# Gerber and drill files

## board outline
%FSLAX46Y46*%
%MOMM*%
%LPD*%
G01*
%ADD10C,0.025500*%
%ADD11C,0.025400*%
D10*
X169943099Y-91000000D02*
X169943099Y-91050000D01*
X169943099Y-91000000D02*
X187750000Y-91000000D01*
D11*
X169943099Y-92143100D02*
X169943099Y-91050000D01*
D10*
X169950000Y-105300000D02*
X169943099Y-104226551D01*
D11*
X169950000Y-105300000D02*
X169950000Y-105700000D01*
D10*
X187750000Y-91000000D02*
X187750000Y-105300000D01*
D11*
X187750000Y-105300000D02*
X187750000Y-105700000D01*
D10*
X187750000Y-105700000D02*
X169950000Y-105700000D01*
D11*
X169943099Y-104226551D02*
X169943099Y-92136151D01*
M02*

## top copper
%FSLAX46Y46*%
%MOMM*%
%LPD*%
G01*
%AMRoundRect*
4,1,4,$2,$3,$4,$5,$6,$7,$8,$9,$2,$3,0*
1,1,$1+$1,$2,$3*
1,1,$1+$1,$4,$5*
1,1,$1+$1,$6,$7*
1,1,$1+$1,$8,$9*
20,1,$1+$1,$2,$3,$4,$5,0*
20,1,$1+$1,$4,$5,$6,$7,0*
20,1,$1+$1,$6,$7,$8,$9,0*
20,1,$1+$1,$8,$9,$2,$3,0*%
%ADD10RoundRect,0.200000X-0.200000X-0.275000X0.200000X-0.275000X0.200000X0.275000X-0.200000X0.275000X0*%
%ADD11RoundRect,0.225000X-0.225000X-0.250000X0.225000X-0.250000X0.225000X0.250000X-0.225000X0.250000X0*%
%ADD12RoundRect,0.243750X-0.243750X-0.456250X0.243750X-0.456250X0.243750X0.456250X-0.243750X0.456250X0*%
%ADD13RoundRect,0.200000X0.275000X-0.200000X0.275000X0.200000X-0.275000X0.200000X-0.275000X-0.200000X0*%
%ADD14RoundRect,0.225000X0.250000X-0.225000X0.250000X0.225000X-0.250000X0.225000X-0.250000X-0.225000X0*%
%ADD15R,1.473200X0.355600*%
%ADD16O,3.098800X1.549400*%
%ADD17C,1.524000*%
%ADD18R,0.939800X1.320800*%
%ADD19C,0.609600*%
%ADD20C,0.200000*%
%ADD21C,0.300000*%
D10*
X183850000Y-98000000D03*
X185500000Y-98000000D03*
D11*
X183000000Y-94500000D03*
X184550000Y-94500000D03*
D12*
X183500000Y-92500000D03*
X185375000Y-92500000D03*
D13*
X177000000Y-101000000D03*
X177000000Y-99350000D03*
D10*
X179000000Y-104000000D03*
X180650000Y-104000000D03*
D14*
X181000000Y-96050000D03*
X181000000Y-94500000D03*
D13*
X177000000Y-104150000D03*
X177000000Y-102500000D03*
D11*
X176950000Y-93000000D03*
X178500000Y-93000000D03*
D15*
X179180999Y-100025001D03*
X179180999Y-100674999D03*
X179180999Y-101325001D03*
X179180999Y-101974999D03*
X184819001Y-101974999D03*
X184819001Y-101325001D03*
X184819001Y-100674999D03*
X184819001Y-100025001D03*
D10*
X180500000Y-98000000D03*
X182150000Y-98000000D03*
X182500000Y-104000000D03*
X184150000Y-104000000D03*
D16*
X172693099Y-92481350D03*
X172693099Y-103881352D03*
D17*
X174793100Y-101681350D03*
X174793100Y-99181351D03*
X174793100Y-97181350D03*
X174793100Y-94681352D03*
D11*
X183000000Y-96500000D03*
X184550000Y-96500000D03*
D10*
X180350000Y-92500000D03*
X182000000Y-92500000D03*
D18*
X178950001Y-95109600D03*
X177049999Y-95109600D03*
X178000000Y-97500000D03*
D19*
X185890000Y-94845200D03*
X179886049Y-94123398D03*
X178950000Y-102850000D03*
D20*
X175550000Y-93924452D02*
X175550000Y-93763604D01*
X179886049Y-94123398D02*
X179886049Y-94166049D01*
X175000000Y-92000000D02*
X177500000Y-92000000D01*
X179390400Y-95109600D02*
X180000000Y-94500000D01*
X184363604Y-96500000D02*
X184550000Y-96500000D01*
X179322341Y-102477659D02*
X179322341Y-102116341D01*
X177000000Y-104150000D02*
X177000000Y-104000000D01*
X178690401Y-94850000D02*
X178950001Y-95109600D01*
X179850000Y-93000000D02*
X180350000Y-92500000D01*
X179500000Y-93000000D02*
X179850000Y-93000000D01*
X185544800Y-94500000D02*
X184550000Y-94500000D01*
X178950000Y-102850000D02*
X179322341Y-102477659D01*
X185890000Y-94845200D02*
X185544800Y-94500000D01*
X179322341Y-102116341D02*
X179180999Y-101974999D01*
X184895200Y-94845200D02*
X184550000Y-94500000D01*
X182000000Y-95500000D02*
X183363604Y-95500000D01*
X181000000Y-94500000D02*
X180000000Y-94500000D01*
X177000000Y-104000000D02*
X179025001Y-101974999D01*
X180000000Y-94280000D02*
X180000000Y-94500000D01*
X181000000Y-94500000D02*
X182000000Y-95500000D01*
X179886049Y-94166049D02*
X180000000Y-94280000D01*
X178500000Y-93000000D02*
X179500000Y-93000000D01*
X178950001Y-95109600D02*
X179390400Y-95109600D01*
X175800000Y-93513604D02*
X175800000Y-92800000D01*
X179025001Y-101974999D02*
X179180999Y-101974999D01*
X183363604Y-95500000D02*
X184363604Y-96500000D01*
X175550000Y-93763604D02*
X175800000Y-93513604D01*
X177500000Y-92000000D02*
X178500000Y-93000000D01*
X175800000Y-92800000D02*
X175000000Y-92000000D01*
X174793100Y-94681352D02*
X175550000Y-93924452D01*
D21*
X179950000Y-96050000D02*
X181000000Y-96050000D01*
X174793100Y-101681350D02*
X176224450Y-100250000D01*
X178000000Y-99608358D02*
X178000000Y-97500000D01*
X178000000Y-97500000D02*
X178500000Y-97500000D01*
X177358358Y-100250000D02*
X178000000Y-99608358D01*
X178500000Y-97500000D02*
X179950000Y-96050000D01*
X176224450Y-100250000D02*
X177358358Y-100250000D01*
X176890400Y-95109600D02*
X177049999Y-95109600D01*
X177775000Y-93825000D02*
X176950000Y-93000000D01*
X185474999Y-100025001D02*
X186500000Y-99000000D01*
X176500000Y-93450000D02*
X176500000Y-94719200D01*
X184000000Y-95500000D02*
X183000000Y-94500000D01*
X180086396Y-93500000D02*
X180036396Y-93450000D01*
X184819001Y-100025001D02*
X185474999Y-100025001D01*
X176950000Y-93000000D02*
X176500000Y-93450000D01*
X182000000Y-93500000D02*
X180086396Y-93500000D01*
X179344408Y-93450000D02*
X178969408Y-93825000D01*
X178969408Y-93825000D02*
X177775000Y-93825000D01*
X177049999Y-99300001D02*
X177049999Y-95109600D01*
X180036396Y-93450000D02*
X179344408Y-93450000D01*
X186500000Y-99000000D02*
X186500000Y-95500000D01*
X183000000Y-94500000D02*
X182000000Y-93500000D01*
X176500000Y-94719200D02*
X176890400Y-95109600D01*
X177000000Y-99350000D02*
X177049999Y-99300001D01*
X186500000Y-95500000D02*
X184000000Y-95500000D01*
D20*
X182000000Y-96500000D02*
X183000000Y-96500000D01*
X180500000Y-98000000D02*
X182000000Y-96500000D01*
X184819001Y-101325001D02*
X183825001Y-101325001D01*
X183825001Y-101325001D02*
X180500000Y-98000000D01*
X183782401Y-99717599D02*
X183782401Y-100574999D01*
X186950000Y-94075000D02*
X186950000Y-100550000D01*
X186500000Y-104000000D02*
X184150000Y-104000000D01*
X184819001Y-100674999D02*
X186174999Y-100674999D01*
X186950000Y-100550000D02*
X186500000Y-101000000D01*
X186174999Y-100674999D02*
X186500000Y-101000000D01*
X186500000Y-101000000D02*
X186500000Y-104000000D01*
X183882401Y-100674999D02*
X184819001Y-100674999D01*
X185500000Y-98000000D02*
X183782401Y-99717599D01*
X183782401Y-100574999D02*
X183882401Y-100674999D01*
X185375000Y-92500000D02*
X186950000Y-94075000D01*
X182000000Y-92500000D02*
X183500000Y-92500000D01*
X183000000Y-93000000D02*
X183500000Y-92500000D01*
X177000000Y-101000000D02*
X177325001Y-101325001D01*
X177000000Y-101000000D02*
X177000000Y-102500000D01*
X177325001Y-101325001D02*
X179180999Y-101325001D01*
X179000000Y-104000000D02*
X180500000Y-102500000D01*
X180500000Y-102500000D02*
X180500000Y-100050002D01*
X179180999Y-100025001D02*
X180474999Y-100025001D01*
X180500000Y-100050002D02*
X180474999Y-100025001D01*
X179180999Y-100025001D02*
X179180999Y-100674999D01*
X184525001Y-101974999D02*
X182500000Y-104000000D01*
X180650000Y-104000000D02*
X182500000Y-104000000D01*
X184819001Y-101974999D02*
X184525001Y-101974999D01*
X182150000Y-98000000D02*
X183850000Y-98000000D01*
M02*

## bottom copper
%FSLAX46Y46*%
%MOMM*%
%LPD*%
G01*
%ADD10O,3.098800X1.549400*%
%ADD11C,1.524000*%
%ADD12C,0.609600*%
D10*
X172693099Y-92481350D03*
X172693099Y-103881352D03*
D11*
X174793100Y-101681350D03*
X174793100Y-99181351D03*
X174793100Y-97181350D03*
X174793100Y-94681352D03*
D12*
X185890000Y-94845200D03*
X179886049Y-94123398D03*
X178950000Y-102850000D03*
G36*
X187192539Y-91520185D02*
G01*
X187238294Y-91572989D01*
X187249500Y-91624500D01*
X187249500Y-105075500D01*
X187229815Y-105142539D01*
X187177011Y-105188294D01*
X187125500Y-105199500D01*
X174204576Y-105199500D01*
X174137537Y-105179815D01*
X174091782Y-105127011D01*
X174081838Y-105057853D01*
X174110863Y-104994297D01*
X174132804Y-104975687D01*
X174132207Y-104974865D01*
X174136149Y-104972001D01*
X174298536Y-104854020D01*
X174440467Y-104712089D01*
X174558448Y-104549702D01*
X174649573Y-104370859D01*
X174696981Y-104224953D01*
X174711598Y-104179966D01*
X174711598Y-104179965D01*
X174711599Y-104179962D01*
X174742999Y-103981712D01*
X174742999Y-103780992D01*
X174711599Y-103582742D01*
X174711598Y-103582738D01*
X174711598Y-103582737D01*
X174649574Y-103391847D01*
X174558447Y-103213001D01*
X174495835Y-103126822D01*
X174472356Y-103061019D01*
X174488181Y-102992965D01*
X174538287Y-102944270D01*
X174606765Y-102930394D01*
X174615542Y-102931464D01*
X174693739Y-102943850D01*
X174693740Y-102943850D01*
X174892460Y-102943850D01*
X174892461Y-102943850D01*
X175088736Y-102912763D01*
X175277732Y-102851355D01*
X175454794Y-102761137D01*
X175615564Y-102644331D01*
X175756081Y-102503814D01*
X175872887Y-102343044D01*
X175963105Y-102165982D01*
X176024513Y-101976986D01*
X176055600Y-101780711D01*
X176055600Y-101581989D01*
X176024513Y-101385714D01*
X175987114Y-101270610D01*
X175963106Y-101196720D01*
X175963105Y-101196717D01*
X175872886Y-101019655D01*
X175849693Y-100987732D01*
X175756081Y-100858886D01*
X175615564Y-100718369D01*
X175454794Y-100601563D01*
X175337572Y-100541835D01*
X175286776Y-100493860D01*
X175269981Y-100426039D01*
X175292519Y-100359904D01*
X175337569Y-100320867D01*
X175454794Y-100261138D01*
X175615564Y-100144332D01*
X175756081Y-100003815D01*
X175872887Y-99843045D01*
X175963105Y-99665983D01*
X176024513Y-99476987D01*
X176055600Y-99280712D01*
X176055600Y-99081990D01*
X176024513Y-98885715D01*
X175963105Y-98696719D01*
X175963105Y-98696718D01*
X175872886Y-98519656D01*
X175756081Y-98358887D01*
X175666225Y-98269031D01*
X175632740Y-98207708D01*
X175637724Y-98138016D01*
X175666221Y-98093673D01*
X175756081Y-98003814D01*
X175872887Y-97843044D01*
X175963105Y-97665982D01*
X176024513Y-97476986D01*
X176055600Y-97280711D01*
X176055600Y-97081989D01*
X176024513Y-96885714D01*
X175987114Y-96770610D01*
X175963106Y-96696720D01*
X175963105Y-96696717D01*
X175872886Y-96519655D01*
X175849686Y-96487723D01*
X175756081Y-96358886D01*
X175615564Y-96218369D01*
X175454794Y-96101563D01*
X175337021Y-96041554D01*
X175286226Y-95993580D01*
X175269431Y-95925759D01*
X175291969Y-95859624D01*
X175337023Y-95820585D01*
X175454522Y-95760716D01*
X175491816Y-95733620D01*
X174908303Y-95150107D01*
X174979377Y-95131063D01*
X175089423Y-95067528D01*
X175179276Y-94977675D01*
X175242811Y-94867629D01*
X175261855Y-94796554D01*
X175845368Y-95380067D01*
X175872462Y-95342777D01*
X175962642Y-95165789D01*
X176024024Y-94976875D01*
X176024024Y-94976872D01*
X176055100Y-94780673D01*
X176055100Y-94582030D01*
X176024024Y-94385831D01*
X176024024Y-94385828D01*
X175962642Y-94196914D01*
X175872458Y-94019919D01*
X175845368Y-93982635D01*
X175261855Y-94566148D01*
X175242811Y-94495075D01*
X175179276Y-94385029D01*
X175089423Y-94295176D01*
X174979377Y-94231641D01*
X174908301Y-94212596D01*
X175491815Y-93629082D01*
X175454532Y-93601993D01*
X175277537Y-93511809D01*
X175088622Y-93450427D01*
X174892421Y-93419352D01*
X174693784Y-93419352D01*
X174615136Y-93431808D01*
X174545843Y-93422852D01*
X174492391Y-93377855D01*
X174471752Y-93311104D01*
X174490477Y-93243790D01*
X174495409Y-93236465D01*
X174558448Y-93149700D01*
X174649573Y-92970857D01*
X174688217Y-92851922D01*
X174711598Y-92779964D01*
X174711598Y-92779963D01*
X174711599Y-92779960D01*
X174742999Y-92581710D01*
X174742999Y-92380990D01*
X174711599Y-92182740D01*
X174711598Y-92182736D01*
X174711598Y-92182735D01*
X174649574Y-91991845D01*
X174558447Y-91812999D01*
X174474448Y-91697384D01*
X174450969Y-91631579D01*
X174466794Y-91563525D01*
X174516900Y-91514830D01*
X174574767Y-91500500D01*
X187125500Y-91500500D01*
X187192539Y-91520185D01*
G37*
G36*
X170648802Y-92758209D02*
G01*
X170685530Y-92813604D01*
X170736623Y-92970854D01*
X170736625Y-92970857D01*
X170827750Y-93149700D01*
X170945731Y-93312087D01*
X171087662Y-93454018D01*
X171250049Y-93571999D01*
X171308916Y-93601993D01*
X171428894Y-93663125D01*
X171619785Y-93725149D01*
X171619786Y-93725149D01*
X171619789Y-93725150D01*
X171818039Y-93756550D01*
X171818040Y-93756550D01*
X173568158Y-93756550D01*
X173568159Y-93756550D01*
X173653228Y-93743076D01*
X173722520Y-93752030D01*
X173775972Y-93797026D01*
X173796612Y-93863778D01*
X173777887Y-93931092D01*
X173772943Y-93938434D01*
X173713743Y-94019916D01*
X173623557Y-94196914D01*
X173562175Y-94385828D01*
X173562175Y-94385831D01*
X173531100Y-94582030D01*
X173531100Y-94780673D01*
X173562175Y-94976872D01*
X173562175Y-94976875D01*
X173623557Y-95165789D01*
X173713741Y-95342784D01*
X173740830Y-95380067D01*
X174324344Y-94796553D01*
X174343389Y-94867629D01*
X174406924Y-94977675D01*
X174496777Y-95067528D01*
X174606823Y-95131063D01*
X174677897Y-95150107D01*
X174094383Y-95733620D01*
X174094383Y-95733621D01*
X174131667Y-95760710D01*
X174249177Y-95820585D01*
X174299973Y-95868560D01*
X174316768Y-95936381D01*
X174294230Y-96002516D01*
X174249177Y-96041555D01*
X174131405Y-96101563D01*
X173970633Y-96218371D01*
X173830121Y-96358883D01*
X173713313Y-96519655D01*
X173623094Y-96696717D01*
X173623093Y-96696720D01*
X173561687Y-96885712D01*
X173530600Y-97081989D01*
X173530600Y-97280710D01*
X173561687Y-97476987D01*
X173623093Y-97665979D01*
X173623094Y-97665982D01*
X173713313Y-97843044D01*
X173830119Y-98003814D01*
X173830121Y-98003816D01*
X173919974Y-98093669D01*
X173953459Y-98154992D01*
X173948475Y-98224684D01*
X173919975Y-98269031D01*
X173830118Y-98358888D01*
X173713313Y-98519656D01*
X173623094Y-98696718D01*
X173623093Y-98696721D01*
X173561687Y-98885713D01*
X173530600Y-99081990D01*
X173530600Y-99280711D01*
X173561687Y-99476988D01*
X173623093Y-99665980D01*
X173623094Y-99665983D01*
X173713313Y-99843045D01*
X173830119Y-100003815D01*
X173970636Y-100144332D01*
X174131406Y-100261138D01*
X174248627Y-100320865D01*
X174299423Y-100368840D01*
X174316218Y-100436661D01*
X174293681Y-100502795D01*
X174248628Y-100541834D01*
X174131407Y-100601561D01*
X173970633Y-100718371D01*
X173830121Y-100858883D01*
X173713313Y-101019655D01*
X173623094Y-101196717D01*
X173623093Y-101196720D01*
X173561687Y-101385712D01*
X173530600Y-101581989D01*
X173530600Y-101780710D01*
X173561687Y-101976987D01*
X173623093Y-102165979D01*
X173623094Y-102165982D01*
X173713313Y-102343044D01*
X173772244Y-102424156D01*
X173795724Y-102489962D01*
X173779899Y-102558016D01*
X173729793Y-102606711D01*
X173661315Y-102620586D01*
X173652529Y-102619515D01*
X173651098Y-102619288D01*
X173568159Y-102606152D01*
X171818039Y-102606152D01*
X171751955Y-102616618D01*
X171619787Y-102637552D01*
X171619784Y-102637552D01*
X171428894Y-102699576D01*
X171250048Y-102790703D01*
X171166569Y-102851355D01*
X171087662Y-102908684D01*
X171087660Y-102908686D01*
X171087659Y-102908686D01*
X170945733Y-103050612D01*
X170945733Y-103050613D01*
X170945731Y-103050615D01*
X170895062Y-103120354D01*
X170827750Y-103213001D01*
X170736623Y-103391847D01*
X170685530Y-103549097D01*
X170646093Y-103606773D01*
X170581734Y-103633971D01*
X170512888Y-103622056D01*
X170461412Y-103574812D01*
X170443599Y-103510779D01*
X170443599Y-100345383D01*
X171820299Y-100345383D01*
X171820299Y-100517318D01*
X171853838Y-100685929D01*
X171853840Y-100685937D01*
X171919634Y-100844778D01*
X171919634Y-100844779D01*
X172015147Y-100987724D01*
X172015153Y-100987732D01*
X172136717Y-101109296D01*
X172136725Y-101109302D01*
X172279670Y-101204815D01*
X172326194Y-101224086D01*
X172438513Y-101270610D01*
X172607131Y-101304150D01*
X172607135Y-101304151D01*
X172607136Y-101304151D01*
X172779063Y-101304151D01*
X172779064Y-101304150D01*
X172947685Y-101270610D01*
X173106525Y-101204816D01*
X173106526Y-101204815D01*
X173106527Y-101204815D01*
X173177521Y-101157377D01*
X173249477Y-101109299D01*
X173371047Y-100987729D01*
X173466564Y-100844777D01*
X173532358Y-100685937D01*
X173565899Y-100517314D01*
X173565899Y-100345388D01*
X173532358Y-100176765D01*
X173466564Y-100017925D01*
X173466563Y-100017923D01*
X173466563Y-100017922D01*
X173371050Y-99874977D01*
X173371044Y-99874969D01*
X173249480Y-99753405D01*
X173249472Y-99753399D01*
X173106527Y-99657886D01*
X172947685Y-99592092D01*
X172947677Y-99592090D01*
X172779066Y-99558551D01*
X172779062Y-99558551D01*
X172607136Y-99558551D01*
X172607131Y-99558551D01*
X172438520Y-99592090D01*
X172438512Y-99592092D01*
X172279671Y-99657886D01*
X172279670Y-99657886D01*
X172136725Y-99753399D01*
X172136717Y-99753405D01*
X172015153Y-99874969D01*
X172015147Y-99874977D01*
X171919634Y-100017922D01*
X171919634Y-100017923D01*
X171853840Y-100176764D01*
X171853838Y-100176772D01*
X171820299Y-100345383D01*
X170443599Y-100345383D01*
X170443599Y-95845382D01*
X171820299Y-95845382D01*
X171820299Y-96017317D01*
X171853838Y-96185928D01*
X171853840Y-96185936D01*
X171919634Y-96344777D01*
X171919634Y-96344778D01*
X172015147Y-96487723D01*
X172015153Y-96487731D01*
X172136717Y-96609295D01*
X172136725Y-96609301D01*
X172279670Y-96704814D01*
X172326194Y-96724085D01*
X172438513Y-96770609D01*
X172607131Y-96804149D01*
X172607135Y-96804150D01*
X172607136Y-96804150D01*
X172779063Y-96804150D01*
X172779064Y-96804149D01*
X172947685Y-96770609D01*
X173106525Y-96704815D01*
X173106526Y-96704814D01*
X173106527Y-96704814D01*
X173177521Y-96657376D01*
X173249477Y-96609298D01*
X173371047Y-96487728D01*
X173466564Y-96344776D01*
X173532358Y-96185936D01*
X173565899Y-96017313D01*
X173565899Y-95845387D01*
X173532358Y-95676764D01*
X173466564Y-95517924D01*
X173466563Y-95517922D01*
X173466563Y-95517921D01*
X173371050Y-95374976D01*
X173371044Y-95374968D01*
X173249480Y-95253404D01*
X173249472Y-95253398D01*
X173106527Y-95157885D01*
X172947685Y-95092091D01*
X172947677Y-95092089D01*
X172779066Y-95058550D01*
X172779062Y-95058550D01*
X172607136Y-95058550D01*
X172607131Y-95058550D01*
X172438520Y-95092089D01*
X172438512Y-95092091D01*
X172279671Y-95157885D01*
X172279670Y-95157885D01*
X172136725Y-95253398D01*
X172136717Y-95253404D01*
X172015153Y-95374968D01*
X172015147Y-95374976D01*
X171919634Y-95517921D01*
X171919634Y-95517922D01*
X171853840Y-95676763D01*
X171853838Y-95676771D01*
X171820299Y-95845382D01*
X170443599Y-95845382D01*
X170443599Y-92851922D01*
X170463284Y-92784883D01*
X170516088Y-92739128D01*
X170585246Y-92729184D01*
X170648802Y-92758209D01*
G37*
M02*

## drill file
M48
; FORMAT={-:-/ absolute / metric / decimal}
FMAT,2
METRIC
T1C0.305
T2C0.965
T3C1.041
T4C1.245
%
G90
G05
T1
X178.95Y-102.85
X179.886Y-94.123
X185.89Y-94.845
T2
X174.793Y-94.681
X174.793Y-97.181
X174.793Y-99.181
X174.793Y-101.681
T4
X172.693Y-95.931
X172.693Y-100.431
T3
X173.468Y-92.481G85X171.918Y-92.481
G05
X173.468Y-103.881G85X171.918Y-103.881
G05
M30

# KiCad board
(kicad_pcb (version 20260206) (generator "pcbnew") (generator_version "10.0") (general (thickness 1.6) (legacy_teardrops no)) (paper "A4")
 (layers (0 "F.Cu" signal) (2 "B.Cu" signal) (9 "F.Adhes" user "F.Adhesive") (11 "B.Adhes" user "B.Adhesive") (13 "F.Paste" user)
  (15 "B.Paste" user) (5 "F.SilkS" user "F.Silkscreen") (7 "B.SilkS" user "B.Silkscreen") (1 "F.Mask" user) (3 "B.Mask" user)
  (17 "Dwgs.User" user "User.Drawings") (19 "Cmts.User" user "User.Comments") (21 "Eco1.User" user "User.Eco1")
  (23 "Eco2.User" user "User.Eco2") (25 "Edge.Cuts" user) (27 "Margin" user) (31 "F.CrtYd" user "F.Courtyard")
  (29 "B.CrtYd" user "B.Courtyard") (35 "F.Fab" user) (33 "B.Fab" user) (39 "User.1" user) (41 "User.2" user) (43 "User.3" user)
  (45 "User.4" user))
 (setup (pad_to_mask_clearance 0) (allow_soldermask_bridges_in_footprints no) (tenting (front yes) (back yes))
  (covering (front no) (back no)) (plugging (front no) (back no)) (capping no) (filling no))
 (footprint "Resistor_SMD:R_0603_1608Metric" (layer "F.Cu") (at 184.675 98)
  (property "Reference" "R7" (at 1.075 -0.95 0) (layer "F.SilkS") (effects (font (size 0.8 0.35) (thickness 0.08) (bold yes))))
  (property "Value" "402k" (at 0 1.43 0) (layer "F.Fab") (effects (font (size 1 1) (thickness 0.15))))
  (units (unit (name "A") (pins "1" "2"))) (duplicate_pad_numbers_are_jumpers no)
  (pad "1" smd roundrect (at -0.825 0) (size 0.8 0.95) (layers "F.Cu" "F.Mask" "F.Paste") (roundrect_rratio 0.25) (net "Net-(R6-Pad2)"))
  (pad "2" smd roundrect (at 0.825 0) (size 0.8 0.95) (layers "F.Cu" "F.Mask" "F.Paste") (roundrect_rratio 0.25) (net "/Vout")))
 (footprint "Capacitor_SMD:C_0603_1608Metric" (layer "F.Cu") (at 183.775 94.5)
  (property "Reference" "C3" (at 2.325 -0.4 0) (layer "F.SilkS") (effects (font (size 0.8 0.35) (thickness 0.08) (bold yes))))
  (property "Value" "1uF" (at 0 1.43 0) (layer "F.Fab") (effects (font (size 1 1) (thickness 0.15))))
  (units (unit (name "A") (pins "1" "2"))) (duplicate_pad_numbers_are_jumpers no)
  (pad "1" smd roundrect (at -0.775 0) (size 0.9 0.95) (layers "F.Cu" "F.Mask" "F.Paste") (roundrect_rratio 0.25) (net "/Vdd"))
  (pad "2" smd roundrect (at 0.775 0) (size 0.9 0.95) (layers "F.Cu" "F.Mask" "F.Paste") (roundrect_rratio 0.25) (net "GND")))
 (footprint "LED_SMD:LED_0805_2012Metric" (layer "F.Cu") (at 184.4375 92.5)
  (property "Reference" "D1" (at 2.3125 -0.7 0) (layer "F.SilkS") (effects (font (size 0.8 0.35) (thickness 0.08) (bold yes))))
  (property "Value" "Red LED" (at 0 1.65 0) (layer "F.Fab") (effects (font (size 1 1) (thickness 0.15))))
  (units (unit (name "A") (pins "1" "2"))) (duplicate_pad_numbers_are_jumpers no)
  (pad "1" smd roundrect (at -0.9375 0) (size 0.975 1.4) (layers "F.Cu" "F.Mask" "F.Paste") (roundrect_rratio 0.25) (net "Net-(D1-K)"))
  (pad "2" smd roundrect (at 0.9375 0) (size 0.975 1.4) (layers "F.Cu" "F.Mask" "F.Paste") (roundrect_rratio 0.25) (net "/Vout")))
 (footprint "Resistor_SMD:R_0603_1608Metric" (layer "F.Cu") (at 177 100.175 90)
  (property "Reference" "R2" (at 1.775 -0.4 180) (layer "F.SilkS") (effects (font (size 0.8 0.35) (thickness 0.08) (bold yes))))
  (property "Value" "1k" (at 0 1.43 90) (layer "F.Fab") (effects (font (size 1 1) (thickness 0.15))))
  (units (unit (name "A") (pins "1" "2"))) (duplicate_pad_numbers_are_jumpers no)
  (pad "1" smd roundrect (at -0.825 0 90) (size 0.8 0.95) (layers "F.Cu" "F.Mask" "F.Paste") (roundrect_rratio 0.25) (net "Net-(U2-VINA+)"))
  (pad "2" smd roundrect (at 0.825 0 90) (size 0.8 0.95) (layers "F.Cu" "F.Mask" "F.Paste") (roundrect_rratio 0.25) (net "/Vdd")))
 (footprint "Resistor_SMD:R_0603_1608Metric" (layer "F.Cu") (at 179.825 104)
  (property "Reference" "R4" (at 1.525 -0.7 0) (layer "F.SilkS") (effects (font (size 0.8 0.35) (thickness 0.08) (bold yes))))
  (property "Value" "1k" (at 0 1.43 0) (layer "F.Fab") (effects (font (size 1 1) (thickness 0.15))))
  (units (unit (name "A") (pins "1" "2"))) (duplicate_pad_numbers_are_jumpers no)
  (pad "1" smd roundrect (at -0.825 0) (size 0.8 0.95) (layers "F.Cu" "F.Mask" "F.Paste") (roundrect_rratio 0.25) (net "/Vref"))
  (pad "2" smd roundrect (at 0.825 0) (size 0.8 0.95) (layers "F.Cu" "F.Mask" "F.Paste") (roundrect_rratio 0.25) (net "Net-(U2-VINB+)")))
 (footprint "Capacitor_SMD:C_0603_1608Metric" (layer "F.Cu") (at 181 95.275 90)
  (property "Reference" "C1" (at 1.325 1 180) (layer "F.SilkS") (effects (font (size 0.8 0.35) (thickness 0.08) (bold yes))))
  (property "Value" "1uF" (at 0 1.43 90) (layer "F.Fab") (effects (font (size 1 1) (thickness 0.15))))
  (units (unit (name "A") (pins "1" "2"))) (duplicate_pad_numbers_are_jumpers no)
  (pad "1" smd roundrect (at -0.775 0 90) (size 0.9 0.95) (layers "F.Cu" "F.Mask" "F.Paste") (roundrect_rratio 0.25) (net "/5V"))
  (pad "2" smd roundrect (at 0.775 0 90) (size 0.9 0.95) (layers "F.Cu" "F.Mask" "F.Paste") (roundrect_rratio 0.25) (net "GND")))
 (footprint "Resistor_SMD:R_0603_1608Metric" (layer "F.Cu") (at 177 103.325 90)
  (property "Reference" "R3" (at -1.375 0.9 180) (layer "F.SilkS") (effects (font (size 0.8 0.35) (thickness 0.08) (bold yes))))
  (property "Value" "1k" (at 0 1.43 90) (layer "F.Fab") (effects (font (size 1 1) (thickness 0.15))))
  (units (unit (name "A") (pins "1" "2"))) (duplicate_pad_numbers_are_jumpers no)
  (pad "1" smd roundrect (at -0.825 0 90) (size 0.8 0.95) (layers "F.Cu" "F.Mask" "F.Paste") (roundrect_rratio 0.25) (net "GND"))
  (pad "2" smd roundrect (at 0.825 0 90) (size 0.8 0.95) (layers "F.Cu" "F.Mask" "F.Paste") (roundrect_rratio 0.25) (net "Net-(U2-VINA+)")))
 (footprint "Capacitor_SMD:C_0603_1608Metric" (layer "F.Cu") (at 177.725 93)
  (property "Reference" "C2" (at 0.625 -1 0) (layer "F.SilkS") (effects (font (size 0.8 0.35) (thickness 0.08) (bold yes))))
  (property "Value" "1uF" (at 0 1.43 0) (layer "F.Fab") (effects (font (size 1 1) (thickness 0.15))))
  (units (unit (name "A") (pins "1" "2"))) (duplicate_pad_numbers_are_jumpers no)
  (pad "1" smd roundrect (at -0.775 0) (size 0.9 0.95) (layers "F.Cu" "F.Mask" "F.Paste") (roundrect_rratio 0.25) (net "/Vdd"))
  (pad "2" smd roundrect (at 0.775 0) (size 0.9 0.95) (layers "F.Cu" "F.Mask" "F.Paste") (roundrect_rratio 0.25) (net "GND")))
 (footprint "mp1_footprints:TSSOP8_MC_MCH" (layer "F.Cu") (at 182 101)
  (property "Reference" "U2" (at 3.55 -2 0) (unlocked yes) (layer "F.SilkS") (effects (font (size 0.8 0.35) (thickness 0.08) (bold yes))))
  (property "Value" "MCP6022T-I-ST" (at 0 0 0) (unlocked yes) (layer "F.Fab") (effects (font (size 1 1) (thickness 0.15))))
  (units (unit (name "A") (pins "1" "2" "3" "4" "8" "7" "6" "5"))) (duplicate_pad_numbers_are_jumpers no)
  (pad "1" smd rect (at -2.819001 -0.974999) (size 1.4732 0.3556) (layers "F.Cu" "F.Mask" "F.Paste") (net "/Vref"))
  (pad "2" smd rect (at -2.819001 -0.325001) (size 1.4732 0.3556) (layers "F.Cu" "F.Mask" "F.Paste") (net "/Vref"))
  (pad "3" smd rect (at -2.819001 0.325001) (size 1.4732 0.3556) (layers "F.Cu" "F.Mask" "F.Paste") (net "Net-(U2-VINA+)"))
  (pad "4" smd rect (at -2.819001 0.974999) (size 1.4732 0.3556) (layers "F.Cu" "F.Mask" "F.Paste") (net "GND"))
  (pad "5" smd rect (at 2.819001 0.974999) (size 1.4732 0.3556) (layers "F.Cu" "F.Mask" "F.Paste") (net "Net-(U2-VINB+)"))
  (pad "6" smd rect (at 2.819001 0.325001) (size 1.4732 0.3556) (layers "F.Cu" "F.Mask" "F.Paste") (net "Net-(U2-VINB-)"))
  (pad "7" smd rect (at 2.819001 -0.325001) (size 1.4732 0.3556) (layers "F.Cu" "F.Mask" "F.Paste") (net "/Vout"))
  (pad "8" smd rect (at 2.819001 -0.974999) (size 1.4732 0.3556) (layers "F.Cu" "F.Mask" "F.Paste") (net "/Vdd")))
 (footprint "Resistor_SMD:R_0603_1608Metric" (layer "F.Cu") (at 181.325 98)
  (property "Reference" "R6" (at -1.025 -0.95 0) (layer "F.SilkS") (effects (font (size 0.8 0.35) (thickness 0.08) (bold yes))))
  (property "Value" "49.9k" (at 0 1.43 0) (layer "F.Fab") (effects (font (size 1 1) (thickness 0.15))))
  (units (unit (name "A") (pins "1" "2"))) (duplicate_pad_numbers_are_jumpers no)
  (pad "1" smd roundrect (at -0.825 0) (size 0.8 0.95) (layers "F.Cu" "F.Mask" "F.Paste") (roundrect_rratio 0.25) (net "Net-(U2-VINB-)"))
  (pad "2" smd roundrect (at 0.825 0) (size 0.8 0.95) (layers "F.Cu" "F.Mask" "F.Paste") (roundrect_rratio 0.25) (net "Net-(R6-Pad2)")))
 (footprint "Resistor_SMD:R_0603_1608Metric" (layer "F.Cu") (at 183.325 104)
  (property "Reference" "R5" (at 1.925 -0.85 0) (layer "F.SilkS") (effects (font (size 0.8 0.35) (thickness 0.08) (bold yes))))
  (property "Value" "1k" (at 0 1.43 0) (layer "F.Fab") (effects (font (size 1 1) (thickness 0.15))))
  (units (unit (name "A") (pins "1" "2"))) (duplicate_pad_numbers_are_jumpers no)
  (pad "1" smd roundrect (at -0.825 0) (size 0.8 0.95) (layers "F.Cu" "F.Mask" "F.Paste") (roundrect_rratio 0.25) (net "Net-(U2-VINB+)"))
  (pad "2" smd roundrect (at 0.825 0) (size 0.8 0.95) (layers "F.Cu" "F.Mask" "F.Paste") (roundrect_rratio 0.25) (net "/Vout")))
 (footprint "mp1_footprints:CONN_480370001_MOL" (layer "F.Cu") (at 174.7931 101.68135 -90)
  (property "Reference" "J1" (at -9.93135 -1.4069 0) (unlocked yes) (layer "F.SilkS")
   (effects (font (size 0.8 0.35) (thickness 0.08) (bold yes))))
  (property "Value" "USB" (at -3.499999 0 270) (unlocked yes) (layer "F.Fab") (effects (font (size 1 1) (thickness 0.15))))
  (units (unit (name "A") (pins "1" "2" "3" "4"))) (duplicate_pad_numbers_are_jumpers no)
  (fp_line (start 2.545201 4.850001) (end -9.545199 4.850001) (stroke (width 0.0254) (type solid)) (layer "Edge.Cuts"))
  (pad "" np_thru_hole oval (at -9.2 2.100001 270) (size 1.5494 3.0988) (drill oval 1.0414 2.5908) (layers "*.Cu" "*.Mask"))
  (pad "" np_thru_hole circle (at -5.75 2.100001 270) (size 1.2446 1.2446) (drill 1.2446) (layers))
  (pad "" np_thru_hole circle (at -1.249999 2.100001 270) (size 1.2446 1.2446) (drill 1.2446) (layers))
  (pad "" np_thru_hole oval (at 2.200002 2.100001 270) (size 1.5494 3.0988) (drill oval 1.0414 2.5908) (layers "*.Cu" "*.Mask"))
  (pad "1" thru_hole circle (at 0 0 270) (size 1.524 1.524) (drill 0.9652) (layers "*.Cu" "*.Mask") (remove_unused_layers no) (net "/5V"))
  (pad "2" thru_hole circle (at -2.499999 0 270) (size 1.524 1.524) (drill 0.9652) (layers "*.Cu" "*.Mask") (remove_unused_layers no)
   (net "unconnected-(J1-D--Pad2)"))
  (pad "3" thru_hole circle (at -4.5 0 270) (size 1.524 1.524) (drill 0.9652) (layers "*.Cu" "*.Mask") (remove_unused_layers no)
   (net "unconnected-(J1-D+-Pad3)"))
  (pad "4" thru_hole circle (at -6.999998 0 270) (size 1.524 1.524) (drill 0.9652) (layers "*.Cu" "*.Mask") (remove_unused_layers no)
   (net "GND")))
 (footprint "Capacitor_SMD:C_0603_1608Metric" (layer "F.Cu") (at 183.775 96.5)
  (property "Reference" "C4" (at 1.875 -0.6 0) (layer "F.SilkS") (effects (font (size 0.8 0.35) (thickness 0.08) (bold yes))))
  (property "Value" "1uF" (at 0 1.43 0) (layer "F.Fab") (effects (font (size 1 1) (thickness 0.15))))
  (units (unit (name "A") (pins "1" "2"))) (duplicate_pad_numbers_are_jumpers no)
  (pad "1" smd roundrect (at -0.775 0) (size 0.9 0.95) (layers "F.Cu" "F.Mask" "F.Paste") (roundrect_rratio 0.25) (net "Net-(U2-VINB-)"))
  (pad "2" smd roundrect (at 0.775 0) (size 0.9 0.95) (layers "F.Cu" "F.Mask" "F.Paste") (roundrect_rratio 0.25) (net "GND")))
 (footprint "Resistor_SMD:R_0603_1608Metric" (layer "F.Cu") (at 181.175 92.5)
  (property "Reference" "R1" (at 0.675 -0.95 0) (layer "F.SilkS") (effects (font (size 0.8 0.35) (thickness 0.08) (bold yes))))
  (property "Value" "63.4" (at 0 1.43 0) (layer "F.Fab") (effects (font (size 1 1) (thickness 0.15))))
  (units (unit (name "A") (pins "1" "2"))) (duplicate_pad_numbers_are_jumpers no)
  (pad "1" smd roundrect (at -0.825 0) (size 0.8 0.95) (layers "F.Cu" "F.Mask" "F.Paste") (roundrect_rratio 0.25) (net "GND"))
  (pad "2" smd roundrect (at 0.825 0) (size 0.8 0.95) (layers "F.Cu" "F.Mask" "F.Paste") (roundrect_rratio 0.25) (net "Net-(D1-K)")))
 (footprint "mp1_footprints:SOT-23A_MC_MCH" (layer "F.Cu") (at 178 96.3048 180)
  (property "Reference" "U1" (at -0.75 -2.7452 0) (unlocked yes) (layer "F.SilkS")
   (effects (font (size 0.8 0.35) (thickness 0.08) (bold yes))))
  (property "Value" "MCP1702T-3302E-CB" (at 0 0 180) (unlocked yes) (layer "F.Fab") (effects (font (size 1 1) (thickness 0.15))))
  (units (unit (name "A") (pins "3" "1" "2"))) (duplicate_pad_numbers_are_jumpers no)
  (pad "1" smd rect (at -0.950001 1.1952 180) (size 0.9398 1.3208) (layers "F.Cu" "F.Mask" "F.Paste") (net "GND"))
  (pad "2" smd rect (at 0.950001 1.1952 180) (size 0.9398 1.3208) (layers "F.Cu" "F.Mask" "F.Paste") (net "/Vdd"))
  (pad "3" smd rect (at 0 -1.1952 180) (size 0.9398 1.3208) (layers "F.Cu" "F.Mask" "F.Paste") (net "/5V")))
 (gr_line (start 169.943099 91) (end 169.943099 91.05) (stroke (width 0.0255) (type solid)) (layer "Edge.Cuts"))
 (gr_line (start 169.943099 91) (end 187.75 91) (stroke (width 0.0255) (type solid)) (layer "Edge.Cuts"))
 (gr_line (start 169.943099 92.1431) (end 169.943099 91.05) (stroke (width 0.0254) (type solid)) (layer "Edge.Cuts"))
 (gr_line (start 169.95 105.3) (end 169.943099 104.226551) (stroke (width 0.0255) (type solid)) (layer "Edge.Cuts"))
 (gr_line (start 169.95 105.3) (end 169.95 105.7) (stroke (width 0.0254) (type solid)) (layer "Edge.Cuts"))
 (gr_line (start 187.75 91) (end 187.75 105.3) (stroke (width 0.0255) (type solid)) (layer "Edge.Cuts"))
 (gr_line (start 187.75 105.3) (end 187.75 105.7) (stroke (width 0.0254) (type solid)) (layer "Edge.Cuts"))
 (gr_line (start 187.75 105.7) (end 169.95 105.7) (stroke (width 0.0255) (type solid)) (layer "Edge.Cuts"))
 (segment (start 175.55 93.924452) (end 175.55 93.763604) (width 0.2) (layer "F.Cu") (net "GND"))
 (segment (start 179.886049 94.123398) (end 179.886049 94.166049) (width 0.2) (layer "F.Cu") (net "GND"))
 (segment (start 175 92) (end 177.5 92) (width 0.2) (layer "F.Cu") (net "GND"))
 (segment (start 179.3904 95.1096) (end 180 94.5) (width 0.2) (layer "F.Cu") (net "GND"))
 (segment (start 184.363604 96.5) (end 184.55 96.5) (width 0.2) (layer "F.Cu") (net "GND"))
 (segment (start 179.322341 102.477659) (end 179.322341 102.116341) (width 0.2) (layer "F.Cu") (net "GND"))
 (segment (start 177 104.15) (end 177 104) (width 0.2) (layer "F.Cu") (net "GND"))
 (segment (start 178.690401 94.85) (end 178.950001 95.1096) (width 0.2) (layer "F.Cu") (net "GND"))
 (segment (start 179.85 93) (end 180.35 92.5) (width 0.2) (layer "F.Cu") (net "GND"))
 (segment (start 179.5 93) (end 179.85 93) (width 0.2) (layer "F.Cu") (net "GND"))
 (segment (start 185.5448 94.5) (end 184.55 94.5) (width 0.2) (layer "F.Cu") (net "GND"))
 (segment (start 178.95 102.85) (end 179.322341 102.477659) (width 0.2) (layer "F.Cu") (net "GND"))
 (segment (start 185.89 94.8452) (end 185.5448 94.5) (width 0.2) (layer "F.Cu") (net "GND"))
 (segment (start 179.322341 102.116341) (end 179.180999 101.974999) (width 0.2) (layer "F.Cu") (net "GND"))
 (segment (start 184.8952 94.8452) (end 184.55 94.5) (width 0.2) (layer "F.Cu") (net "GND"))
 (segment (start 182 95.5) (end 183.363604 95.5) (width 0.2) (layer "F.Cu") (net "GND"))
 (segment (start 181 94.5) (end 180 94.5) (width 0.2) (layer "F.Cu") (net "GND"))
 (segment (start 177 104) (end 179.025001 101.974999) (width 0.2) (layer "F.Cu") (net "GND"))
 (segment (start 180 94.28) (end 180 94.5) (width 0.2) (layer "F.Cu") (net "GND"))
 (segment (start 181 94.5) (end 182 95.5) (width 0.2) (layer "F.Cu") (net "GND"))
 (segment (start 179.886049 94.166049) (end 180 94.28) (width 0.2) (layer "F.Cu") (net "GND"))
 (segment (start 178.5 93) (end 179.5 93) (width 0.2) (layer "F.Cu") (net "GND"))
 (segment (start 178.950001 95.1096) (end 179.3904 95.1096) (width 0.2) (layer "F.Cu") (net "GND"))
 (segment (start 175.8 93.513604) (end 175.8 92.8) (width 0.2) (layer "F.Cu") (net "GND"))
 (segment (start 179.025001 101.974999) (end 179.180999 101.974999) (width 0.2) (layer "F.Cu") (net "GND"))
 (segment (start 183.363604 95.5) (end 184.363604 96.5) (width 0.2) (layer "F.Cu") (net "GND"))
 (segment (start 175.55 93.763604) (end 175.8 93.513604) (width 0.2) (layer "F.Cu") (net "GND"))
 (segment (start 177.5 92) (end 178.5 93) (width 0.2) (layer "F.Cu") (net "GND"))
 (segment (start 175.8 92.8) (end 175 92) (width 0.2) (layer "F.Cu") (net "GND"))
 (segment (start 174.7931 94.681352) (end 175.55 93.924452) (width 0.2) (layer "F.Cu") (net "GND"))
 (via (at 185.89 94.8452) (size 0.6096) (drill 0.3048) (layers "F.Cu" "B.Cu") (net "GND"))
 (via (at 179.886049 94.123398) (size 0.6096) (drill 0.3048) (layers "F.Cu" "B.Cu") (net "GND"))
 (via (at 178.95 102.85) (size 0.6096) (drill 0.3048) (layers "F.Cu" "B.Cu") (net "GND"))
 (segment (start 179.95 96.05) (end 181 96.05) (width 0.3) (layer "F.Cu") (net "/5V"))
 (segment (start 174.7931 101.68135) (end 176.22445 100.25) (width 0.3) (layer "F.Cu") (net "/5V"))
 (segment (start 178 99.608358) (end 178 97.5) (width 0.3) (layer "F.Cu") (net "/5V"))
 (segment (start 178 97.5) (end 178.5 97.5) (width 0.3) (layer "F.Cu") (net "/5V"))
 (segment (start 177.358358 100.25) (end 178 99.608358) (width 0.3) (layer "F.Cu") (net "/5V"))
 (segment (start 178.5 97.5) (end 179.95 96.05) (width 0.3) (layer "F.Cu") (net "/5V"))
 (segment (start 176.22445 100.25) (end 177.358358 100.25) (width 0.3) (layer "F.Cu") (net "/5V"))
 (segment (start 176.8904 95.1096) (end 177.049999 95.1096) (width 0.3) (layer "F.Cu") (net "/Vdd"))
 (segment (start 177.775 93.825) (end 176.95 93) (width 0.3) (layer "F.Cu") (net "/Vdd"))
 (segment (start 185.474999 100.025001) (end 186.5 99) (width 0.3) (layer "F.Cu") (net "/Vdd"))
 (segment (start 176.5 93.45) (end 176.5 94.7192) (width 0.3) (layer "F.Cu") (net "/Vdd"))
 (segment (start 184 95.5) (end 183 94.5) (width 0.3) (layer "F.Cu") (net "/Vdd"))
 (segment (start 180.086396 93.5) (end 180.036396 93.45) (width 0.3) (layer "F.Cu") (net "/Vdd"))
 (segment (start 184.819001 100.025001) (end 185.474999 100.025001) (width 0.3) (layer "F.Cu") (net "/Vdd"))
 (segment (start 176.95 93) (end 176.5 93.45) (width 0.3) (layer "F.Cu") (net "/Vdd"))
 (segment (start 182 93.5) (end 180.086396 93.5) (width 0.3) (layer "F.Cu") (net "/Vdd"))
 (segment (start 179.344408 93.45) (end 178.969408 93.825) (width 0.3) (layer "F.Cu") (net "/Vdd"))
 (segment (start 178.969408 93.825) (end 177.775 93.825) (width 0.3) (layer "F.Cu") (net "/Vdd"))
 (segment (start 177.049999 99.300001) (end 177.049999 95.1096) (width 0.3) (layer "F.Cu") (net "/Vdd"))
 (segment (start 180.036396 93.45) (end 179.344408 93.45) (width 0.3) (layer "F.Cu") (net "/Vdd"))
 (segment (start 186.5 99) (end 186.5 95.5) (width 0.3) (layer "F.Cu") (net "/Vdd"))
 (segment (start 183 94.5) (end 182 93.5) (width 0.3) (layer "F.Cu") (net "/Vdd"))
 (segment (start 176.5 94.7192) (end 176.8904 95.1096) (width 0.3) (layer "F.Cu") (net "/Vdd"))
 (segment (start 177 99.35) (end 177.049999 99.300001) (width 0.3) (layer "F.Cu") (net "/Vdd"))
 (segment (start 186.5 95.5) (end 184 95.5) (width 0.3) (layer "F.Cu") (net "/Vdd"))
 (segment (start 182 96.5) (end 183 96.5) (width 0.2) (layer "F.Cu") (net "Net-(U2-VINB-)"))
 (segment (start 180.5 98) (end 182 96.5) (width 0.2) (layer "F.Cu") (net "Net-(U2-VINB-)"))
 (segment (start 184.819001 101.325001) (end 183.825001 101.325001) (width 0.2) (layer "F.Cu") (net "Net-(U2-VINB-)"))
 (segment (start 183.825001 101.325001) (end 180.5 98) (width 0.2) (layer "F.Cu") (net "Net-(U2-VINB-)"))
 (segment (start 183.782401 99.717599) (end 183.782401 100.574999) (width 0.2) (layer "F.Cu") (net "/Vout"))
 (segment (start 186.95 94.075) (end 186.95 100.55) (width 0.2) (layer "F.Cu") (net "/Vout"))
 (segment (start 186.5 104) (end 184.15 104) (width 0.2) (layer "F.Cu") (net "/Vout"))
 (segment (start 184.819001 100.674999) (end 186.174999 100.674999) (width 0.2) (layer "F.Cu") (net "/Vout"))
 (segment (start 186.95 100.55) (end 186.5 101) (width 0.2) (layer "F.Cu") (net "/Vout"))
 (segment (start 186.174999 100.674999) (end 186.5 101) (width 0.2) (layer "F.Cu") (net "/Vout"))
 (segment (start 186.5 101) (end 186.5 104) (width 0.2) (layer "F.Cu") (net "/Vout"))
 (segment (start 183.882401 100.674999) (end 184.819001 100.674999) (width 0.2) (layer "F.Cu") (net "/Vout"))
 (segment (start 185.5 98) (end 183.782401 99.717599) (width 0.2) (layer "F.Cu") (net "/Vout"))
 (segment (start 183.782401 100.574999) (end 183.882401 100.674999) (width 0.2) (layer "F.Cu") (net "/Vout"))
 (segment (start 185.375 92.5) (end 186.95 94.075) (width 0.2) (layer "F.Cu") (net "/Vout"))
 (segment (start 182 92.5) (end 183.5 92.5) (width 0.2) (layer "F.Cu") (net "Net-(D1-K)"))
 (segment (start 183 93) (end 183.5 92.5) (width 0.2) (layer "F.Cu") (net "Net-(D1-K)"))
 (segment (start 177 101) (end 177.325001 101.325001) (width 0.2) (layer "F.Cu") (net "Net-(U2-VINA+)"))
 (segment (start 177 101) (end 177 102.5) (width 0.2) (layer "F.Cu") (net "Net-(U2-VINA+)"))
 (segment (start 177.325001 101.325001) (end 179.180999 101.325001) (width 0.2) (layer "F.Cu") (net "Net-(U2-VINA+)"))
 (segment (start 179 104) (end 180.5 102.5) (width 0.2) (layer "F.Cu") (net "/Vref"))
 (segment (start 180.5 102.5) (end 180.5 100.050002) (width 0.2) (layer "F.Cu") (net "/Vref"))
 (segment (start 179.180999 100.025001) (end 180.474999 100.025001) (width 0.2) (layer "F.Cu") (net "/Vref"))
 (segment (start 180.5 100.050002) (end 180.474999 100.025001) (width 0.2) (layer "F.Cu") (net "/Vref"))
 (segment (start 179.180999 100.025001) (end 179.180999 100.674999) (width 0.2) (layer "F.Cu") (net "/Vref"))
 (segment (start 184.525001 101.974999) (end 182.5 104) (width 0.2) (layer "F.Cu") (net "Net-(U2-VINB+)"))
 (segment (start 180.65 104) (end 182.5 104) (width 0.2) (layer "F.Cu") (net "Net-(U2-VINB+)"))
 (segment (start 184.819001 101.974999) (end 184.525001 101.974999) (width 0.2) (layer "F.Cu") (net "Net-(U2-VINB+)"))
 (segment (start 182.15 98) (end 183.85 98) (width 0.2) (layer "F.Cu") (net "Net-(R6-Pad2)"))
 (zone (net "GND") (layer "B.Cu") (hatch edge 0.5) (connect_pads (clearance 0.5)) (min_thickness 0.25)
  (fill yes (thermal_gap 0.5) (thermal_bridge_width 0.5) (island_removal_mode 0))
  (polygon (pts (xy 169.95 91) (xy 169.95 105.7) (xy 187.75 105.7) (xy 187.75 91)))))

